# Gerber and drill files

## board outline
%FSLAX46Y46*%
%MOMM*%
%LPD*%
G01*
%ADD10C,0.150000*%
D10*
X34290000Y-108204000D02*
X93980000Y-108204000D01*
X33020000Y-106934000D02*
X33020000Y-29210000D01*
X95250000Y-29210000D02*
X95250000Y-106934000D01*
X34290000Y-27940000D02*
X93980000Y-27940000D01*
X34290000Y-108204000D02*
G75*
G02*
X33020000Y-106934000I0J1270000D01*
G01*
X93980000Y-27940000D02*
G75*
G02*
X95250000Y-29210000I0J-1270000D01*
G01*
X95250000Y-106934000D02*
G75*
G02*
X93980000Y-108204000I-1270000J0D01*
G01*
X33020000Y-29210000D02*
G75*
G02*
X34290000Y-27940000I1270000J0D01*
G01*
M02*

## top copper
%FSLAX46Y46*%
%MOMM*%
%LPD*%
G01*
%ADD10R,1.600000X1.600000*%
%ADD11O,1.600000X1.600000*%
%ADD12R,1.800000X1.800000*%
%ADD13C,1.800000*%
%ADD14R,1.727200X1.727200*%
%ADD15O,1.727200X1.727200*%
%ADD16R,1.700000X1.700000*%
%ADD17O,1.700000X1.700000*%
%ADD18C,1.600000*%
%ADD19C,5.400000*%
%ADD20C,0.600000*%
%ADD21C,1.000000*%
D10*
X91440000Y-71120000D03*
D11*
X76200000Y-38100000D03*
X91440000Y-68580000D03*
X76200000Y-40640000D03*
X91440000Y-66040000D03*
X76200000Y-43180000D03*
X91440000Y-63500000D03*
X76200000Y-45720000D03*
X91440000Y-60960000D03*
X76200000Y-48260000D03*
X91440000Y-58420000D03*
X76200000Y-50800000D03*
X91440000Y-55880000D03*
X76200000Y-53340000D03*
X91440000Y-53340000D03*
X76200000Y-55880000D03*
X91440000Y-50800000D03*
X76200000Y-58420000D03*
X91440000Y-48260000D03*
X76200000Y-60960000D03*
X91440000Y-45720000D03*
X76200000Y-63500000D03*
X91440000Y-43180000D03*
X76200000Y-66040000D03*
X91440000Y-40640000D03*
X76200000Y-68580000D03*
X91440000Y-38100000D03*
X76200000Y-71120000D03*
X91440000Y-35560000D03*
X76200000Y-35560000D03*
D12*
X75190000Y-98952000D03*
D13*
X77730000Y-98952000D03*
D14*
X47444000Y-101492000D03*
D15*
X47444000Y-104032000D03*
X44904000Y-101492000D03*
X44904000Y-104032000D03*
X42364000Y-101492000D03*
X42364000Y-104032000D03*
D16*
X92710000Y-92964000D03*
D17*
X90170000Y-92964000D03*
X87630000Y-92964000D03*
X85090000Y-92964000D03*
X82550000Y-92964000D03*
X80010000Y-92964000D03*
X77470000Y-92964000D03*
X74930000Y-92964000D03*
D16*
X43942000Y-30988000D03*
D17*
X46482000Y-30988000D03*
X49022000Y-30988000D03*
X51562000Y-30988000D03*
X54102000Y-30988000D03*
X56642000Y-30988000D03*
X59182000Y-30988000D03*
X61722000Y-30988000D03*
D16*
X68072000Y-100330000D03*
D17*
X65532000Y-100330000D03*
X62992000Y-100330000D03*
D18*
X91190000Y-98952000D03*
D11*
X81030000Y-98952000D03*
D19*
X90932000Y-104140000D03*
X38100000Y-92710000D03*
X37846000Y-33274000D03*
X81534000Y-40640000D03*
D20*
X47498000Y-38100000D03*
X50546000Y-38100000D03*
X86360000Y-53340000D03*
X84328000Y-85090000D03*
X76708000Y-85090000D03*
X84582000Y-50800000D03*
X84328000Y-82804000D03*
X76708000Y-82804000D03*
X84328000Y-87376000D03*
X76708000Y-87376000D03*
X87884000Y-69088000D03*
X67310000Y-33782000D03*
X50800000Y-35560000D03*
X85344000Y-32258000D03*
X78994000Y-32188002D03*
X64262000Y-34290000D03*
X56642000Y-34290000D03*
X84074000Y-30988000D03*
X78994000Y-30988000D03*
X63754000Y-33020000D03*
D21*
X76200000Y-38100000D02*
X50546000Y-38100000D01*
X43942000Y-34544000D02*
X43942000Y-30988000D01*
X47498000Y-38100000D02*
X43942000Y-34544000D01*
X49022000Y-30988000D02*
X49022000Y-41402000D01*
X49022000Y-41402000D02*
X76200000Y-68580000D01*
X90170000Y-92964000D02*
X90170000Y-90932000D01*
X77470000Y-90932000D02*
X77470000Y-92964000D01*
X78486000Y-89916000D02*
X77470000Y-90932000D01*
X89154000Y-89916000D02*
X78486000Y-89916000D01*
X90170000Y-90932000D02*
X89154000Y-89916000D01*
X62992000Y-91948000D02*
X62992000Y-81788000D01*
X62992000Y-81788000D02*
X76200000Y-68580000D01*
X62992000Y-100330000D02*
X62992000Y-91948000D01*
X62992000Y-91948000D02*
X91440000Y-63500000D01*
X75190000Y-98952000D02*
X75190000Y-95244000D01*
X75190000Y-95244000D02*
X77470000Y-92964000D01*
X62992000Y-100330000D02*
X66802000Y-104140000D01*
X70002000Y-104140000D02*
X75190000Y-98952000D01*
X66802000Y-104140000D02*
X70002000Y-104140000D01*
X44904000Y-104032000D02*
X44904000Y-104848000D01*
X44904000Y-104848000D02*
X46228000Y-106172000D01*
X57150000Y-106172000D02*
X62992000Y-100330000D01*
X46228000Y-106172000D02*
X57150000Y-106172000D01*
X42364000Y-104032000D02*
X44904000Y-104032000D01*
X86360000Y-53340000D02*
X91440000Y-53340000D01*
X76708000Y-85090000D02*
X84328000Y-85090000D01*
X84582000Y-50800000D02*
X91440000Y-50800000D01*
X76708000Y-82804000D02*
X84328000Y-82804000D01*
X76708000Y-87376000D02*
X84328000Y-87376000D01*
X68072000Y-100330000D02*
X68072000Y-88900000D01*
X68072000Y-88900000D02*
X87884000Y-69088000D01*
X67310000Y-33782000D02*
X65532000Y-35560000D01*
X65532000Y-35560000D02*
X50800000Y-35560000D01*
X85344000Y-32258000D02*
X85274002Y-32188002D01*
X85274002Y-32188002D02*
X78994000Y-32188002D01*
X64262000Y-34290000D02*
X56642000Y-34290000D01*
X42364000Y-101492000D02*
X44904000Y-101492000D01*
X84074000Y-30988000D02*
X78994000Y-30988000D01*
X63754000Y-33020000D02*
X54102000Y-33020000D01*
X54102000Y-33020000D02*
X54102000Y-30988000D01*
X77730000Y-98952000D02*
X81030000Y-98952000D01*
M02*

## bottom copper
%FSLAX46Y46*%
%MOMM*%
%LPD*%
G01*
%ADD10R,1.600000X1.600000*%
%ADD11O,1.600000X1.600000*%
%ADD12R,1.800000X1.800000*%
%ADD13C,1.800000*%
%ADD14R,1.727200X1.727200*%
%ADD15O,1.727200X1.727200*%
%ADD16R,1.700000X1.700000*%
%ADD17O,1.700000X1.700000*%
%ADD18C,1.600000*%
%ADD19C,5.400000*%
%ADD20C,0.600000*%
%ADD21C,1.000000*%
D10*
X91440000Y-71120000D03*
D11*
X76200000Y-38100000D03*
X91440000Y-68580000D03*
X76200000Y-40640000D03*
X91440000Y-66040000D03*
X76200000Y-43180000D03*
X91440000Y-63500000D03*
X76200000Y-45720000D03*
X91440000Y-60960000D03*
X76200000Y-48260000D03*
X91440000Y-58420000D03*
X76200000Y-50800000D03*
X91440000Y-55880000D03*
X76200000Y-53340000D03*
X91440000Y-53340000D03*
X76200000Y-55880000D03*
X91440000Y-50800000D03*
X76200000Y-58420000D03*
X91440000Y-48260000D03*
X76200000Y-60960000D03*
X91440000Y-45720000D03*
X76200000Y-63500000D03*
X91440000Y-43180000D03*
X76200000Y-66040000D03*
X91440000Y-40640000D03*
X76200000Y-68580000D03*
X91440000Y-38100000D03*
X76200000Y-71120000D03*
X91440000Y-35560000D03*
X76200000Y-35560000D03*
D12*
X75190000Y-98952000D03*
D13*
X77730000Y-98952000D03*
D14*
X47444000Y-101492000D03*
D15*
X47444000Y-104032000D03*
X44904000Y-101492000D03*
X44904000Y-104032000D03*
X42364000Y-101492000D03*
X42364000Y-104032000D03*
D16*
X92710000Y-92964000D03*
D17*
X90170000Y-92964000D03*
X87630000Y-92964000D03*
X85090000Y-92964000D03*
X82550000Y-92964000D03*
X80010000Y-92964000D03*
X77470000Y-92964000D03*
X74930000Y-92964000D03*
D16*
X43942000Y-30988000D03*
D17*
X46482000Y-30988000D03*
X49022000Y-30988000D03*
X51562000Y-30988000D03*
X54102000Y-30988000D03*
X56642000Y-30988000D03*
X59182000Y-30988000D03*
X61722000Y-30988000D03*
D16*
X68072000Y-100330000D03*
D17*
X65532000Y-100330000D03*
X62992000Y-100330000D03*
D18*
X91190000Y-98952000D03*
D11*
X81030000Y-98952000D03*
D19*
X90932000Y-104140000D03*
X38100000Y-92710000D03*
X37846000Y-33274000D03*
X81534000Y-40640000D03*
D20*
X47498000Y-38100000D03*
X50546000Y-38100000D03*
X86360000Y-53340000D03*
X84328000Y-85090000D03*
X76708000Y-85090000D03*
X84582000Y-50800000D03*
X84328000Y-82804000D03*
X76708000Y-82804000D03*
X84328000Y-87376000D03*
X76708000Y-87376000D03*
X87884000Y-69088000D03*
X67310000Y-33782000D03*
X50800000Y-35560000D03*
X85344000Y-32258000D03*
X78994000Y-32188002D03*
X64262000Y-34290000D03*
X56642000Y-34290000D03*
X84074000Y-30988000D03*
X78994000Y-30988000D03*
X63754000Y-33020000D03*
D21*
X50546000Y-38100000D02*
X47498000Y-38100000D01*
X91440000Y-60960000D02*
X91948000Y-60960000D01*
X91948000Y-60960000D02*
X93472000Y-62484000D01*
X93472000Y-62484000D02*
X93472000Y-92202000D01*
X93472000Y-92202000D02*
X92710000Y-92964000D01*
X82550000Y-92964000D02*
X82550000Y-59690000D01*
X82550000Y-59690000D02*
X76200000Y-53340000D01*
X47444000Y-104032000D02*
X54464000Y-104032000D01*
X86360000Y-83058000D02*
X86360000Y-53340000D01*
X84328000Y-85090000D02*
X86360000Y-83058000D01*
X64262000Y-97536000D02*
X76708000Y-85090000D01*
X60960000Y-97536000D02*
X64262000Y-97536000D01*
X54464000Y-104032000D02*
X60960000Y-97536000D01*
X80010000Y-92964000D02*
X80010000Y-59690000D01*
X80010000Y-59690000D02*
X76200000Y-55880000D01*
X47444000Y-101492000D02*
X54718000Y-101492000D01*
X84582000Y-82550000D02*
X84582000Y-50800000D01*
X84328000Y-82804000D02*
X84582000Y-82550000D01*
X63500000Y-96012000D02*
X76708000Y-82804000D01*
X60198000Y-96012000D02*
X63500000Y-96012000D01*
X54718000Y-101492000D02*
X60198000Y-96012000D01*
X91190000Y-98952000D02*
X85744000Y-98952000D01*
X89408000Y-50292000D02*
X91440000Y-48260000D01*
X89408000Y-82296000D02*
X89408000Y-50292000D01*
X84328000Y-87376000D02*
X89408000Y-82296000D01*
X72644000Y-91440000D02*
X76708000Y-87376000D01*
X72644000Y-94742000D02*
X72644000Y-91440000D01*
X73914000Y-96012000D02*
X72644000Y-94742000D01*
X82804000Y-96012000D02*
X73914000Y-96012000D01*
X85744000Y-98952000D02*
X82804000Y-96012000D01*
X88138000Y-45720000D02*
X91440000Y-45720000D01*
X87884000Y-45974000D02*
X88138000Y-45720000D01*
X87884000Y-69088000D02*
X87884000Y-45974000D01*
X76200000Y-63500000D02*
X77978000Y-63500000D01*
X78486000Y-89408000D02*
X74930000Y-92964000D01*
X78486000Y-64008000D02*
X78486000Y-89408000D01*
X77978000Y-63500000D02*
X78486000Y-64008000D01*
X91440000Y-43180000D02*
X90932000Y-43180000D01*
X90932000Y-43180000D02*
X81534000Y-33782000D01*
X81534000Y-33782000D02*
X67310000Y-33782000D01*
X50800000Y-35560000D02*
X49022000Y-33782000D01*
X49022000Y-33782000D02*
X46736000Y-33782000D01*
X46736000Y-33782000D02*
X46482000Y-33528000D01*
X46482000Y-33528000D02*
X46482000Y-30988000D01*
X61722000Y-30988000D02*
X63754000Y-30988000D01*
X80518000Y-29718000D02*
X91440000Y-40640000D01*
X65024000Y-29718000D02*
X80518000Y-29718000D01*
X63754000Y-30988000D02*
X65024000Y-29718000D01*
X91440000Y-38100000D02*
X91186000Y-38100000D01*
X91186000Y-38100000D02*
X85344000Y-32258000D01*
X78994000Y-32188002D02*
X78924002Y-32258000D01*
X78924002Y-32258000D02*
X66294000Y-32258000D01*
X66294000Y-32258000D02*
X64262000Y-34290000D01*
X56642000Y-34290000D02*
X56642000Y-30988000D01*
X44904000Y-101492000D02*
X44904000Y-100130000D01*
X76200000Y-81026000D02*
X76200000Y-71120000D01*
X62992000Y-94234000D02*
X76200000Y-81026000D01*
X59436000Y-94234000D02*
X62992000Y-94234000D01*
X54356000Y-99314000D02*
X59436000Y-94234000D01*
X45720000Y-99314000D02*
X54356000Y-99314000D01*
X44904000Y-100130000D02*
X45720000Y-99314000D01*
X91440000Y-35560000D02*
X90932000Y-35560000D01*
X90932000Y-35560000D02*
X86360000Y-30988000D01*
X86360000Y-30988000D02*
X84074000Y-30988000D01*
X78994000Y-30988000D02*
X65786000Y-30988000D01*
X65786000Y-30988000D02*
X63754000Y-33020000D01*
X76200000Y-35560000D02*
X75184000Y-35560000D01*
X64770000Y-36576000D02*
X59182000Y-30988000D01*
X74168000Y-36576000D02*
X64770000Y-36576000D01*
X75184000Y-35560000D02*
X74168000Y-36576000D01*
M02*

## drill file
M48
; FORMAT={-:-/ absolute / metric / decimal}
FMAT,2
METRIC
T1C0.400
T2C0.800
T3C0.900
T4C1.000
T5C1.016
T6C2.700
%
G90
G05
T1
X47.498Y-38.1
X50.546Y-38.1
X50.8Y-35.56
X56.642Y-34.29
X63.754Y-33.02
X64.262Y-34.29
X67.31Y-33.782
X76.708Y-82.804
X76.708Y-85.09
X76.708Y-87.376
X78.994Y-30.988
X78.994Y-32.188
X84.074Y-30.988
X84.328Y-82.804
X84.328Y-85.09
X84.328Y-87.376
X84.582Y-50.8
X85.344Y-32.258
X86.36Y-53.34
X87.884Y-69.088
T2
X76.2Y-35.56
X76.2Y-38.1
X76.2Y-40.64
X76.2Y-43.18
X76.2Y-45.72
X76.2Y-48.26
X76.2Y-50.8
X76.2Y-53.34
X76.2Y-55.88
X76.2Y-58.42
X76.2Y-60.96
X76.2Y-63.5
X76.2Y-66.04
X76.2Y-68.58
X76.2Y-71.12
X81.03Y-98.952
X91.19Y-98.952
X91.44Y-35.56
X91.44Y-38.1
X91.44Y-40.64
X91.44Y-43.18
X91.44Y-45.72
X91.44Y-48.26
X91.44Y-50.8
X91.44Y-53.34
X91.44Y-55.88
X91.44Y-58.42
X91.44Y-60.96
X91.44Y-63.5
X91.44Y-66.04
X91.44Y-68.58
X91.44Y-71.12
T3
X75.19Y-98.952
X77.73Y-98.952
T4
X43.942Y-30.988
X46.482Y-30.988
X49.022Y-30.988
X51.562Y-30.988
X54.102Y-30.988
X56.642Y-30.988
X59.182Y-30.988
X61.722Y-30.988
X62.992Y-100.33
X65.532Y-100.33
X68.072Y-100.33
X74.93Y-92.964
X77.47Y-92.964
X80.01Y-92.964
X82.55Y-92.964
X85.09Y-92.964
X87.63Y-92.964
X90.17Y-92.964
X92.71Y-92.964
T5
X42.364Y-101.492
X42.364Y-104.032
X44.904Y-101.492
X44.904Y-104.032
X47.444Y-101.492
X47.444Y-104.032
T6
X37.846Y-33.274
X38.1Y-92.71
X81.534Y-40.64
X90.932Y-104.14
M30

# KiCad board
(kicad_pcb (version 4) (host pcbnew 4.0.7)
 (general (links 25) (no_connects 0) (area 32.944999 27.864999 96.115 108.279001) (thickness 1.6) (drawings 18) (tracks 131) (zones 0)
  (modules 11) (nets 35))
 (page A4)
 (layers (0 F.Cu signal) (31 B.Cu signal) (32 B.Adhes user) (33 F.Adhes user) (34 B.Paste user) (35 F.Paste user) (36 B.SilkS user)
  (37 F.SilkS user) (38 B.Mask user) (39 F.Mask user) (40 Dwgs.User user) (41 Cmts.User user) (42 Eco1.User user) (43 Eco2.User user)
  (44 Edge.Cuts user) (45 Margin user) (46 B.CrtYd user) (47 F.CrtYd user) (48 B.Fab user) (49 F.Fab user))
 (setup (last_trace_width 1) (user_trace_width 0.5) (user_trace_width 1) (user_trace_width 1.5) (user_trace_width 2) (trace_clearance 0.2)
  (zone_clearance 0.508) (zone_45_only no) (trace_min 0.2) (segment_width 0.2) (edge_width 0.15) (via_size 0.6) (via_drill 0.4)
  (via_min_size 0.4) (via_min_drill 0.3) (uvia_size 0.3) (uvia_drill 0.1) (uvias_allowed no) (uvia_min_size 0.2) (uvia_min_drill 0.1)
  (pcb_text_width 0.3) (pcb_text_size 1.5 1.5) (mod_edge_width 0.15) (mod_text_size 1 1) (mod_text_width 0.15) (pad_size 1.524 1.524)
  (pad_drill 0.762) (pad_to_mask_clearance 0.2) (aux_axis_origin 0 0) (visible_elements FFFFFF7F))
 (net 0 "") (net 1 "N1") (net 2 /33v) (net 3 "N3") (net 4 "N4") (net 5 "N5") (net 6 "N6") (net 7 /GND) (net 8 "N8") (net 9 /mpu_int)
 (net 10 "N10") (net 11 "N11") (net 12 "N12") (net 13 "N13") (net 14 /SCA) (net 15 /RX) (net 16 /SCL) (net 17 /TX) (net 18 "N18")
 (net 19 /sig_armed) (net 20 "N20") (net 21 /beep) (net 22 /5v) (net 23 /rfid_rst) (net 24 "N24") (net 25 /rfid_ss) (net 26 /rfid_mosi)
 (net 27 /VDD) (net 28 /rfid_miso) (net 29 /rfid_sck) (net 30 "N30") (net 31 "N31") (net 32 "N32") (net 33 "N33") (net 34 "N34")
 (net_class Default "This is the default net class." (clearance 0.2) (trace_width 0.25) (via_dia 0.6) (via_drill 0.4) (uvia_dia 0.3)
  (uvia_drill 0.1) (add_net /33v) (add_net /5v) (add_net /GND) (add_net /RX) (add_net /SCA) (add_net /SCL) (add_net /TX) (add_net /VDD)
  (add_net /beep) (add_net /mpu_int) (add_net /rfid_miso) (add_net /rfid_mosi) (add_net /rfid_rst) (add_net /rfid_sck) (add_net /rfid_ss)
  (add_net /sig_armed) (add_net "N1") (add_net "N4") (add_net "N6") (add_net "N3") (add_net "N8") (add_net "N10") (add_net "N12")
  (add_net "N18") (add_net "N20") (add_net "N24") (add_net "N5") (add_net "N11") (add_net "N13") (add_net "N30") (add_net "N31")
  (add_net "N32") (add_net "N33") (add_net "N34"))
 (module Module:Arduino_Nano (layer F.Cu) (at 91.44 71.12 180)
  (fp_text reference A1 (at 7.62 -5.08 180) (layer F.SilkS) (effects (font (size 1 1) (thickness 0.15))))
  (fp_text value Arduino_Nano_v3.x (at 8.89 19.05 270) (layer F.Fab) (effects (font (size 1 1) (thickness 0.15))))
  (pad 1 thru_hole rect (at 0 0 180) (size 1.6 1.6) (drill 0.8) (layers *.Cu *.Mask) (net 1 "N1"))
  (pad 17 thru_hole oval (at 15.24 33.02 180) (size 1.6 1.6) (drill 0.8) (layers *.Cu *.Mask) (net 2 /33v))
  (pad 2 thru_hole oval (at 0 2.54 180) (size 1.6 1.6) (drill 0.8) (layers *.Cu *.Mask) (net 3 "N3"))
  (pad 18 thru_hole oval (at 15.24 30.48 180) (size 1.6 1.6) (drill 0.8) (layers *.Cu *.Mask) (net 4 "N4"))
  (pad 3 thru_hole oval (at 0 5.08 180) (size 1.6 1.6) (drill 0.8) (layers *.Cu *.Mask) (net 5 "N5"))
  (pad 19 thru_hole oval (at 15.24 27.94 180) (size 1.6 1.6) (drill 0.8) (layers *.Cu *.Mask) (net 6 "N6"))
  (pad 4 thru_hole oval (at 0 7.62 180) (size 1.6 1.6) (drill 0.8) (layers *.Cu *.Mask) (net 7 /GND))
  (pad 20 thru_hole oval (at 15.24 25.4 180) (size 1.6 1.6) (drill 0.8) (layers *.Cu *.Mask) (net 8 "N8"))
  (pad 5 thru_hole oval (at 0 10.16 180) (size 1.6 1.6) (drill 0.8) (layers *.Cu *.Mask) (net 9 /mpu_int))
  (pad 21 thru_hole oval (at 15.24 22.86 180) (size 1.6 1.6) (drill 0.8) (layers *.Cu *.Mask) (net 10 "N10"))
  (pad 6 thru_hole oval (at 0 12.7 180) (size 1.6 1.6) (drill 0.8) (layers *.Cu *.Mask) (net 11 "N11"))
  (pad 22 thru_hole oval (at 15.24 20.32 180) (size 1.6 1.6) (drill 0.8) (layers *.Cu *.Mask) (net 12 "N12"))
  (pad 7 thru_hole oval (at 0 15.24 180) (size 1.6 1.6) (drill 0.8) (layers *.Cu *.Mask) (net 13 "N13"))
  (pad 23 thru_hole oval (at 15.24 17.78 180) (size 1.6 1.6) (drill 0.8) (layers *.Cu *.Mask) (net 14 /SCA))
  (pad 8 thru_hole oval (at 0 17.78 180) (size 1.6 1.6) (drill 0.8) (layers *.Cu *.Mask) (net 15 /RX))
  (pad 24 thru_hole oval (at 15.24 15.24 180) (size 1.6 1.6) (drill 0.8) (layers *.Cu *.Mask) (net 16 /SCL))
  (pad 9 thru_hole oval (at 0 20.32 180) (size 1.6 1.6) (drill 0.8) (layers *.Cu *.Mask) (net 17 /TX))
  (pad 25 thru_hole oval (at 15.24 12.7 180) (size 1.6 1.6) (drill 0.8) (layers *.Cu *.Mask) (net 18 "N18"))
  (pad 10 thru_hole oval (at 0 22.86 180) (size 1.6 1.6) (drill 0.8) (layers *.Cu *.Mask) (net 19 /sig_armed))
  (pad 26 thru_hole oval (at 15.24 10.16 180) (size 1.6 1.6) (drill 0.8) (layers *.Cu *.Mask) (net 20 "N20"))
  (pad 11 thru_hole oval (at 0 25.4 180) (size 1.6 1.6) (drill 0.8) (layers *.Cu *.Mask) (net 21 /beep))
  (pad 27 thru_hole oval (at 15.24 7.62 180) (size 1.6 1.6) (drill 0.8) (layers *.Cu *.Mask) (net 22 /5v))
  (pad 12 thru_hole oval (at 0 27.94 180) (size 1.6 1.6) (drill 0.8) (layers *.Cu *.Mask) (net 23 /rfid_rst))
  (pad 28 thru_hole oval (at 15.24 5.08 180) (size 1.6 1.6) (drill 0.8) (layers *.Cu *.Mask) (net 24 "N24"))
  (pad 13 thru_hole oval (at 0 30.48 180) (size 1.6 1.6) (drill 0.8) (layers *.Cu *.Mask) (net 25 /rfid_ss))
  (pad 29 thru_hole oval (at 15.24 2.54 180) (size 1.6 1.6) (drill 0.8) (layers *.Cu *.Mask) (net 7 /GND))
  (pad 14 thru_hole oval (at 0 33.02 180) (size 1.6 1.6) (drill 0.8) (layers *.Cu *.Mask) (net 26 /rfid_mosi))
  (pad 30 thru_hole oval (at 15.24 0 180) (size 1.6 1.6) (drill 0.8) (layers *.Cu *.Mask) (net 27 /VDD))
  (pad 15 thru_hole oval (at 0 35.56 180) (size 1.6 1.6) (drill 0.8) (layers *.Cu *.Mask) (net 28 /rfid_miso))
  (pad 16 thru_hole oval (at 15.24 35.56 180) (size 1.6 1.6) (drill 0.8) (layers *.Cu *.Mask) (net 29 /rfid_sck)))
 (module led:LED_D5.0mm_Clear (layer F.Cu) (at 75.19 98.952)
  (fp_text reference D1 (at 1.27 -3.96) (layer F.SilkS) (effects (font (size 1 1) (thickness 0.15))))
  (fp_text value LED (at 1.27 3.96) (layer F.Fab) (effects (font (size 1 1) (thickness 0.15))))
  (pad 1 thru_hole rect (at 0 0) (size 1.8 1.8) (drill 0.9) (layers *.Cu *.Mask) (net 7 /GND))
  (pad 2 thru_hole circle (at 2.54 0) (size 1.8 1.8) (drill 0.9) (layers *.Cu *.Mask) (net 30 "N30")))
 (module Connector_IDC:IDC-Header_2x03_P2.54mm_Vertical (layer F.Cu) (at 47.444 101.492 270)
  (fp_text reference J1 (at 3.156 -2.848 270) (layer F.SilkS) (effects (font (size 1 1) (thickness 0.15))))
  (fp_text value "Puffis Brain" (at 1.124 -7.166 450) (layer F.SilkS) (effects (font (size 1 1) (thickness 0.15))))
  (pad 1 thru_hole rect (at 0 0 270) (size 1.7272 1.7272) (drill 1.016) (layers *.Cu *.Mask) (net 17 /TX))
  (pad 2 thru_hole oval (at 2.54 0 270) (size 1.7272 1.7272) (drill 1.016) (layers *.Cu *.Mask) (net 15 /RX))
  (pad 3 thru_hole oval (at 0 2.54 270) (size 1.7272 1.7272) (drill 1.016) (layers *.Cu *.Mask) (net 27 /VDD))
  (pad 4 thru_hole oval (at 2.54 2.54 270) (size 1.7272 1.7272) (drill 1.016) (layers *.Cu *.Mask) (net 7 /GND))
  (pad 5 thru_hole oval (at 0 5.08 270) (size 1.7272 1.7272) (drill 1.016) (layers *.Cu *.Mask) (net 27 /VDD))
  (pad 6 thru_hole oval (at 2.54 5.08 270) (size 1.7272 1.7272) (drill 1.016) (layers *.Cu *.Mask) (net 7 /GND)))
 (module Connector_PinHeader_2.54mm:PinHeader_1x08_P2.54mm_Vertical (layer F.Cu) (at 92.71 92.964 270)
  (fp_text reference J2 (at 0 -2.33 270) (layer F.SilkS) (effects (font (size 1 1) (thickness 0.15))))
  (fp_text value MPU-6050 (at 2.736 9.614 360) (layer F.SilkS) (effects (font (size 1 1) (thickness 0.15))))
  (pad 1 thru_hole rect (at 0 0 270) (size 1.7 1.7) (drill 1) (layers *.Cu *.Mask) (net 9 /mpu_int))
  (pad 2 thru_hole oval (at 0 2.54 270) (size 1.7 1.7) (drill 1) (layers *.Cu *.Mask) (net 7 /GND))
  (pad 3 thru_hole oval (at 0 5.08 270) (size 1.7 1.7) (drill 1) (layers *.Cu *.Mask) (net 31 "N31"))
  (pad 4 thru_hole oval (at 0 7.62 270) (size 1.7 1.7) (drill 1) (layers *.Cu *.Mask) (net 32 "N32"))
  (pad 5 thru_hole oval (at 0 10.16 270) (size 1.7 1.7) (drill 1) (layers *.Cu *.Mask) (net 14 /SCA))
  (pad 6 thru_hole oval (at 0 12.7 270) (size 1.7 1.7) (drill 1) (layers *.Cu *.Mask) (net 16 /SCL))
  (pad 7 thru_hole oval (at 0 15.24 270) (size 1.7 1.7) (drill 1) (layers *.Cu *.Mask) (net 7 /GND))
  (pad 8 thru_hole oval (at 0 17.78 270) (size 1.7 1.7) (drill 1) (layers *.Cu *.Mask) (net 22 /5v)))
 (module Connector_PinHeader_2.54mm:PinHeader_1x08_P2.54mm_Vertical (layer F.Cu) (at 43.942 30.988 90)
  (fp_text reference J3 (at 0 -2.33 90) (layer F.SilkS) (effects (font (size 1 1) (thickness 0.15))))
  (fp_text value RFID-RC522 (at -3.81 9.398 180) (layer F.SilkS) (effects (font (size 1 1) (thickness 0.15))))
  (pad 1 thru_hole rect (at 0 0 90) (size 1.7 1.7) (drill 1) (layers *.Cu *.Mask) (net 2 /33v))
  (pad 2 thru_hole oval (at 0 2.54 90) (size 1.7 1.7) (drill 1) (layers *.Cu *.Mask) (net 23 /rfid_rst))
  (pad 3 thru_hole oval (at 0 5.08 90) (size 1.7 1.7) (drill 1) (layers *.Cu *.Mask) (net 7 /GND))
  (pad 4 thru_hole oval (at 0 7.62 90) (size 1.7 1.7) (drill 1) (layers *.Cu *.Mask) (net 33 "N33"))
  (pad 5 thru_hole oval (at 0 10.16 90) (size 1.7 1.7) (drill 1) (layers *.Cu *.Mask) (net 28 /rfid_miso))
  (pad 6 thru_hole oval (at 0 12.7 90) (size 1.7 1.7) (drill 1) (layers *.Cu *.Mask) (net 26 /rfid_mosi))
  (pad 7 thru_hole oval (at 0 15.24 90) (size 1.7 1.7) (drill 1) (layers *.Cu *.Mask) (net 29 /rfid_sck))
  (pad 8 thru_hole oval (at 0 17.78 90) (size 1.7 1.7) (drill 1) (layers *.Cu *.Mask) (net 25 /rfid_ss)))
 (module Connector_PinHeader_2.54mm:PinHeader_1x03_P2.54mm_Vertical (layer F.Cu) (at 68.072 100.33 270)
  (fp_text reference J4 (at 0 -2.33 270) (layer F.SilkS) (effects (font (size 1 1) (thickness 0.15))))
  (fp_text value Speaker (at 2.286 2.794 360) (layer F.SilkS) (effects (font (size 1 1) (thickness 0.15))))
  (pad 1 thru_hole rect (at 0 0 270) (size 1.7 1.7) (drill 1) (layers *.Cu *.Mask) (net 21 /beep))
  (pad 2 thru_hole oval (at 0 2.54 270) (size 1.7 1.7) (drill 1) (layers *.Cu *.Mask) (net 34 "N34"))
  (pad 3 thru_hole oval (at 0 5.08 270) (size 1.7 1.7) (drill 1) (layers *.Cu *.Mask) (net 7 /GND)))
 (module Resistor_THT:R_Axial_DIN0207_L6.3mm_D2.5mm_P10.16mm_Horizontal (layer F.Cu) (at 91.19 98.952 180)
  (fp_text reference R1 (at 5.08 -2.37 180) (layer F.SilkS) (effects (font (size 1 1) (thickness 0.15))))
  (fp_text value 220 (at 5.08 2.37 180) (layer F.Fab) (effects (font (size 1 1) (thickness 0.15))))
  (pad 1 thru_hole circle (at 0 0 180) (size 1.6 1.6) (drill 0.8) (layers *.Cu *.Mask) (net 19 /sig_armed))
  (pad 2 thru_hole oval (at 10.16 0 180) (size 1.6 1.6) (drill 0.8) (layers *.Cu *.Mask) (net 30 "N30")))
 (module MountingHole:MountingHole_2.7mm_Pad (layer F.Cu) (at 90.932 104.14)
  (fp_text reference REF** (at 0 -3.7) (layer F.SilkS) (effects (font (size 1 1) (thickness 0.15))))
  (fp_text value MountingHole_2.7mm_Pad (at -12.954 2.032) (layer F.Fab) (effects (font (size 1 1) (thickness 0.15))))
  (pad 1 thru_hole circle (at 0 0) (size 5.4 5.4) (drill 2.7) (layers *.Cu *.Mask)))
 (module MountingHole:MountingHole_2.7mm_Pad (layer F.Cu) (at 38.1 92.71)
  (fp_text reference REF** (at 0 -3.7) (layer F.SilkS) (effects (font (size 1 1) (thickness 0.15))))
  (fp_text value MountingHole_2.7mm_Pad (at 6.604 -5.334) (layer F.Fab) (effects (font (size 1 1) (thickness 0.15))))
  (pad 1 thru_hole circle (at 0 0) (size 5.4 5.4) (drill 2.7) (layers *.Cu *.Mask)))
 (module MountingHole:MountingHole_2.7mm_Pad (layer F.Cu) (at 37.846 33.274)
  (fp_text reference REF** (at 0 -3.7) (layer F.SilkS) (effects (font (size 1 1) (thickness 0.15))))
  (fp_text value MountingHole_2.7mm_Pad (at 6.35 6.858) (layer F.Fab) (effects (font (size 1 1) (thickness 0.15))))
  (pad 1 thru_hole circle (at 0 0) (size 5.4 5.4) (drill 2.7) (layers *.Cu *.Mask)))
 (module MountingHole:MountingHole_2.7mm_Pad (layer F.Cu) (at 81.534 40.64)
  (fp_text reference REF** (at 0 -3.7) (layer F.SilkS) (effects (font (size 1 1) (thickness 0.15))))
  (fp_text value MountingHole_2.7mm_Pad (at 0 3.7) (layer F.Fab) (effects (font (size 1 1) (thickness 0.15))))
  (pad 1 thru_hole circle (at 0 0) (size 5.4 5.4) (drill 2.7) (layers *.Cu *.Mask)))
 (gr_line (start 34.29 108.204) (end 93.98 108.204) (angle 90) (layer Edge.Cuts) (width 0.15))
 (gr_line (start 33.02 106.934) (end 33.02 29.21) (angle 90) (layer Edge.Cuts) (width 0.15))
 (gr_line (start 95.25 29.21) (end 95.25 106.934) (angle 90) (layer Edge.Cuts) (width 0.15))
 (gr_line (start 34.29 27.94) (end 93.98 27.94) (angle 90) (layer Edge.Cuts) (width 0.15))
 (gr_arc (start 34.29 106.934) (end 34.29 108.204) (angle 90) (layer Edge.Cuts) (width 0.15))
 (gr_arc (start 93.98 29.21) (end 93.98 27.94) (angle 90) (layer Edge.Cuts) (width 0.15))
 (gr_arc (start 93.98 106.934) (end 95.25 106.934) (angle 90) (layer Edge.Cuts) (width 0.15))
 (gr_arc (start 34.29 29.21) (end 33.02 29.21) (angle 90) (layer Edge.Cuts) (width 0.15))
 (segment (start 76.2 38.1) (end 50.546 38.1) (width 1) (layer F.Cu) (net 2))
 (segment (start 43.942 34.544) (end 43.942 30.988) (width 1) (layer F.Cu) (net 2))
 (segment (start 47.498 38.1) (end 43.942 34.544) (width 1) (layer F.Cu) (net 2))
 (via (at 47.498 38.1) (size 0.6) (drill 0.4) (layers F.Cu B.Cu) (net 2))
 (segment (start 50.546 38.1) (end 47.498 38.1) (width 1) (layer B.Cu) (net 2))
 (via (at 50.546 38.1) (size 0.6) (drill 0.4) (layers F.Cu B.Cu) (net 2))
 (segment (start 49.022 30.988) (end 49.022 41.402) (width 1) (layer F.Cu) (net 7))
 (segment (start 49.022 41.402) (end 76.2 68.58) (width 1) (layer F.Cu) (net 7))
 (segment (start 90.17 92.964) (end 90.17 90.932) (width 1) (layer F.Cu) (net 7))
 (segment (start 77.47 90.932) (end 77.47 92.964) (width 1) (layer F.Cu) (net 7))
 (segment (start 78.486 89.916) (end 77.47 90.932) (width 1) (layer F.Cu) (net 7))
 (segment (start 89.154 89.916) (end 78.486 89.916) (width 1) (layer F.Cu) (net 7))
 (segment (start 90.17 90.932) (end 89.154 89.916) (width 1) (layer F.Cu) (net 7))
 (segment (start 62.992 91.948) (end 62.992 81.788) (width 1) (layer F.Cu) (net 7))
 (segment (start 62.992 81.788) (end 76.2 68.58) (width 1) (layer F.Cu) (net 7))
 (segment (start 62.992 100.33) (end 62.992 91.948) (width 1) (layer F.Cu) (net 7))
 (segment (start 62.992 91.948) (end 91.44 63.5) (width 1) (layer F.Cu) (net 7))
 (segment (start 75.19 98.952) (end 75.19 95.244) (width 1) (layer F.Cu) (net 7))
 (segment (start 75.19 95.244) (end 77.47 92.964) (width 1) (layer F.Cu) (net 7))
 (segment (start 62.992 100.33) (end 66.802 104.14) (width 1) (layer F.Cu) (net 7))
 (segment (start 70.002 104.14) (end 75.19 98.952) (width 1) (layer F.Cu) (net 7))
 (segment (start 66.802 104.14) (end 70.002 104.14) (width 1) (layer F.Cu) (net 7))
 (segment (start 44.904 104.032) (end 44.904 104.848) (width 1) (layer F.Cu) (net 7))
 (segment (start 44.904 104.848) (end 46.228 106.172) (width 1) (layer F.Cu) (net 7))
 (segment (start 57.15 106.172) (end 62.992 100.33) (width 1) (layer F.Cu) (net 7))
 (segment (start 46.228 106.172) (end 57.15 106.172) (width 1) (layer F.Cu) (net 7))
 (segment (start 42.364 104.032) (end 44.904 104.032) (width 1) (layer F.Cu) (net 7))
 (segment (start 91.44 60.96) (end 91.948 60.96) (width 1) (layer B.Cu) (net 9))
 (segment (start 91.948 60.96) (end 93.472 62.484) (width 1) (layer B.Cu) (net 9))
 (segment (start 93.472 62.484) (end 93.472 92.202) (width 1) (layer B.Cu) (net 9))
 (segment (start 93.472 92.202) (end 92.71 92.964) (width 1) (layer B.Cu) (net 9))
 (segment (start 82.55 92.964) (end 82.55 59.69) (width 1) (layer B.Cu) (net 14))
 (segment (start 82.55 59.69) (end 76.2 53.34) (width 1) (layer B.Cu) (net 14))
 (segment (start 47.444 104.032) (end 54.464 104.032) (width 1) (layer B.Cu) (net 15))
 (segment (start 86.36 53.34) (end 91.44 53.34) (width 1) (layer F.Cu) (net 15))
 (via (at 86.36 53.34) (size 0.6) (drill 0.4) (layers F.Cu B.Cu) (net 15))
 (segment (start 86.36 83.058) (end 86.36 53.34) (width 1) (layer B.Cu) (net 15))
 (segment (start 84.328 85.09) (end 86.36 83.058) (width 1) (layer B.Cu) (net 15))
 (via (at 84.328 85.09) (size 0.6) (drill 0.4) (layers F.Cu B.Cu) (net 15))
 (segment (start 76.708 85.09) (end 84.328 85.09) (width 1) (layer F.Cu) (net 15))
 (via (at 76.708 85.09) (size 0.6) (drill 0.4) (layers F.Cu B.Cu) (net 15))
 (segment (start 64.262 97.536) (end 76.708 85.09) (width 1) (layer B.Cu) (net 15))
 (segment (start 60.96 97.536) (end 64.262 97.536) (width 1) (layer B.Cu) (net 15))
 (segment (start 54.464 104.032) (end 60.96 97.536) (width 1) (layer B.Cu) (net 15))
 (segment (start 80.01 92.964) (end 80.01 59.69) (width 1) (layer B.Cu) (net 16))
 (segment (start 80.01 59.69) (end 76.2 55.88) (width 1) (layer B.Cu) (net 16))
 (segment (start 47.444 101.492) (end 54.718 101.492) (width 1) (layer B.Cu) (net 17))
 (segment (start 84.582 50.8) (end 91.44 50.8) (width 1) (layer F.Cu) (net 17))
 (via (at 84.582 50.8) (size 0.6) (drill 0.4) (layers F.Cu B.Cu) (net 17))
 (segment (start 84.582 82.55) (end 84.582 50.8) (width 1) (layer B.Cu) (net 17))
 (segment (start 84.328 82.804) (end 84.582 82.55) (width 1) (layer B.Cu) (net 17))
 (via (at 84.328 82.804) (size 0.6) (drill 0.4) (layers F.Cu B.Cu) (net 17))
 (segment (start 76.708 82.804) (end 84.328 82.804) (width 1) (layer F.Cu) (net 17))
 (via (at 76.708 82.804) (size 0.6) (drill 0.4) (layers F.Cu B.Cu) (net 17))
 (segment (start 63.5 96.012) (end 76.708 82.804) (width 1) (layer B.Cu) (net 17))
 (segment (start 60.198 96.012) (end 63.5 96.012) (width 1) (layer B.Cu) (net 17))
 (segment (start 54.718 101.492) (end 60.198 96.012) (width 1) (layer B.Cu) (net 17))
 (segment (start 91.19 98.952) (end 85.744 98.952) (width 1) (layer B.Cu) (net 19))
 (segment (start 89.408 50.292) (end 91.44 48.26) (width 1) (layer B.Cu) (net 19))
 (segment (start 89.408 82.296) (end 89.408 50.292) (width 1) (layer B.Cu) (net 19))
 (segment (start 84.328 87.376) (end 89.408 82.296) (width 1) (layer B.Cu) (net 19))
 (via (at 84.328 87.376) (size 0.6) (drill 0.4) (layers F.Cu B.Cu) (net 19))
 (segment (start 76.708 87.376) (end 84.328 87.376) (width 1) (layer F.Cu) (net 19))
 (via (at 76.708 87.376) (size 0.6) (drill 0.4) (layers F.Cu B.Cu) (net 19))
 (segment (start 72.644 91.44) (end 76.708 87.376) (width 1) (layer B.Cu) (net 19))
 (segment (start 72.644 94.742) (end 72.644 91.44) (width 1) (layer B.Cu) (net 19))
 (segment (start 73.914 96.012) (end 72.644 94.742) (width 1) (layer B.Cu) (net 19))
 (segment (start 82.804 96.012) (end 73.914 96.012) (width 1) (layer B.Cu) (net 19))
 (segment (start 85.744 98.952) (end 82.804 96.012) (width 1) (layer B.Cu) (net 19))
 (segment (start 68.072 100.33) (end 68.072 88.9) (width 1) (layer F.Cu) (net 21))
 (segment (start 88.138 45.72) (end 91.44 45.72) (width 1) (layer B.Cu) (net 21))
 (segment (start 87.884 45.974) (end 88.138 45.72) (width 1) (layer B.Cu) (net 21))
 (segment (start 87.884 69.088) (end 87.884 45.974) (width 1) (layer B.Cu) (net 21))
 (via (at 87.884 69.088) (size 0.6) (drill 0.4) (layers F.Cu B.Cu) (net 21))
 (segment (start 68.072 88.9) (end 87.884 69.088) (width 1) (layer F.Cu) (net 21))
 (segment (start 76.2 63.5) (end 77.978 63.5) (width 1) (layer B.Cu) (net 22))
 (segment (start 78.486 89.408) (end 74.93 92.964) (width 1) (layer B.Cu) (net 22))
 (segment (start 78.486 64.008) (end 78.486 89.408) (width 1) (layer B.Cu) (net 22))
 (segment (start 77.978 63.5) (end 78.486 64.008) (width 1) (layer B.Cu) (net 22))
 (segment (start 91.44 43.18) (end 90.932 43.18) (width 1) (layer B.Cu) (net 23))
 (segment (start 90.932 43.18) (end 81.534 33.782) (width 1) (layer B.Cu) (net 23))
 (segment (start 81.534 33.782) (end 67.31 33.782) (width 1) (layer B.Cu) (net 23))
 (via (at 67.31 33.782) (size 0.6) (drill 0.4) (layers F.Cu B.Cu) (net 23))
 (segment (start 67.31 33.782) (end 65.532 35.56) (width 1) (layer F.Cu) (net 23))
 (segment (start 65.532 35.56) (end 50.8 35.56) (width 1) (layer F.Cu) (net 23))
 (via (at 50.8 35.56) (size 0.6) (drill 0.4) (layers F.Cu B.Cu) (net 23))
 (segment (start 50.8 35.56) (end 49.022 33.782) (width 1) (layer B.Cu) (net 23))
 (segment (start 49.022 33.782) (end 46.736 33.782) (width 1) (layer B.Cu) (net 23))
 (segment (start 46.736 33.782) (end 46.482 33.528) (width 1) (layer B.Cu) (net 23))
 (segment (start 46.482 33.528) (end 46.482 30.988) (width 1) (layer B.Cu) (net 23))
 (segment (start 61.722 30.988) (end 63.754 30.988) (width 1) (layer B.Cu) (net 25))
 (segment (start 80.518 29.718) (end 91.44 40.64) (width 1) (layer B.Cu) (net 25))
 (segment (start 65.024 29.718) (end 80.518 29.718) (width 1) (layer B.Cu) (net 25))
 (segment (start 63.754 30.988) (end 65.024 29.718) (width 1) (layer B.Cu) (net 25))
 (segment (start 91.44 38.1) (end 91.186 38.1) (width 1) (layer B.Cu) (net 26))
 (segment (start 91.186 38.1) (end 85.344 32.258) (width 1) (layer B.Cu) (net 26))
 (via (at 85.344 32.258) (size 0.6) (drill 0.4) (layers F.Cu B.Cu) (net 26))
 (segment (start 85.344 32.258) (end 85.274002 32.188002) (width 1) (layer F.Cu) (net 26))
 (segment (start 85.274002 32.188002) (end 78.994 32.188002) (width 1) (layer F.Cu) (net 26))
 (via (at 78.994 32.188002) (size 0.6) (drill 0.4) (layers F.Cu B.Cu) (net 26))
 (segment (start 78.994 32.188002) (end 78.924002 32.258) (width 1) (layer B.Cu) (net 26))
 (segment (start 78.924002 32.258) (end 66.294 32.258) (width 1) (layer B.Cu) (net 26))
 (segment (start 66.294 32.258) (end 64.262 34.29) (width 1) (layer B.Cu) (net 26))
 (via (at 64.262 34.29) (size 0.6) (drill 0.4) (layers F.Cu B.Cu) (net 26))
 (segment (start 64.262 34.29) (end 56.642 34.29) (width 1) (layer F.Cu) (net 26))
 (via (at 56.642 34.29) (size 0.6) (drill 0.4) (layers F.Cu B.Cu) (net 26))
 (segment (start 56.642 34.29) (end 56.642 30.988) (width 1) (layer B.Cu) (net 26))
 (segment (start 44.904 101.492) (end 44.904 100.13) (width 1) (layer B.Cu) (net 27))
 (segment (start 76.2 81.026) (end 76.2 71.12) (width 1) (layer B.Cu) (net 27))
 (segment (start 62.992 94.234) (end 76.2 81.026) (width 1) (layer B.Cu) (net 27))
 (segment (start 59.436 94.234) (end 62.992 94.234) (width 1) (layer B.Cu) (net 27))
 (segment (start 54.356 99.314) (end 59.436 94.234) (width 1) (layer B.Cu) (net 27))
 (segment (start 45.72 99.314) (end 54.356 99.314) (width 1) (layer B.Cu) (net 27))
 (segment (start 44.904 100.13) (end 45.72 99.314) (width 1) (layer B.Cu) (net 27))
 (segment (start 42.364 101.492) (end 44.904 101.492) (width 1) (layer F.Cu) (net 27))
 (segment (start 91.44 35.56) (end 90.932 35.56) (width 1) (layer B.Cu) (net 28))
 (segment (start 90.932 35.56) (end 86.36 30.988) (width 1) (layer B.Cu) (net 28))
 (segment (start 86.36 30.988) (end 84.074 30.988) (width 1) (layer B.Cu) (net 28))
 (via (at 84.074 30.988) (size 0.6) (drill 0.4) (layers F.Cu B.Cu) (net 28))
 (segment (start 84.074 30.988) (end 78.994 30.988) (width 1) (layer F.Cu) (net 28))
 (via (at 78.994 30.988) (size 0.6) (drill 0.4) (layers F.Cu B.Cu) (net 28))
 (segment (start 78.994 30.988) (end 65.786 30.988) (width 1) (layer B.Cu) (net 28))
 (segment (start 65.786 30.988) (end 63.754 33.02) (width 1) (layer B.Cu) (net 28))
 (via (at 63.754 33.02) (size 0.6) (drill 0.4) (layers F.Cu B.Cu) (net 28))
 (segment (start 63.754 33.02) (end 54.102 33.02) (width 1) (layer F.Cu) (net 28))
 (segment (start 54.102 33.02) (end 54.102 30.988) (width 1) (layer F.Cu) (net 28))
 (segment (start 76.2 35.56) (end 75.184 35.56) (width 1) (layer B.Cu) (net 29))
 (segment (start 64.77 36.576) (end 59.182 30.988) (width 1) (layer B.Cu) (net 29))
 (segment (start 74.168 36.576) (end 64.77 36.576) (width 1) (layer B.Cu) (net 29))
 (segment (start 75.184 35.56) (end 74.168 36.576) (width 1) (layer B.Cu) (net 29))
 (segment (start 77.73 98.952) (end 81.03 98.952) (width 1) (layer F.Cu) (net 30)))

